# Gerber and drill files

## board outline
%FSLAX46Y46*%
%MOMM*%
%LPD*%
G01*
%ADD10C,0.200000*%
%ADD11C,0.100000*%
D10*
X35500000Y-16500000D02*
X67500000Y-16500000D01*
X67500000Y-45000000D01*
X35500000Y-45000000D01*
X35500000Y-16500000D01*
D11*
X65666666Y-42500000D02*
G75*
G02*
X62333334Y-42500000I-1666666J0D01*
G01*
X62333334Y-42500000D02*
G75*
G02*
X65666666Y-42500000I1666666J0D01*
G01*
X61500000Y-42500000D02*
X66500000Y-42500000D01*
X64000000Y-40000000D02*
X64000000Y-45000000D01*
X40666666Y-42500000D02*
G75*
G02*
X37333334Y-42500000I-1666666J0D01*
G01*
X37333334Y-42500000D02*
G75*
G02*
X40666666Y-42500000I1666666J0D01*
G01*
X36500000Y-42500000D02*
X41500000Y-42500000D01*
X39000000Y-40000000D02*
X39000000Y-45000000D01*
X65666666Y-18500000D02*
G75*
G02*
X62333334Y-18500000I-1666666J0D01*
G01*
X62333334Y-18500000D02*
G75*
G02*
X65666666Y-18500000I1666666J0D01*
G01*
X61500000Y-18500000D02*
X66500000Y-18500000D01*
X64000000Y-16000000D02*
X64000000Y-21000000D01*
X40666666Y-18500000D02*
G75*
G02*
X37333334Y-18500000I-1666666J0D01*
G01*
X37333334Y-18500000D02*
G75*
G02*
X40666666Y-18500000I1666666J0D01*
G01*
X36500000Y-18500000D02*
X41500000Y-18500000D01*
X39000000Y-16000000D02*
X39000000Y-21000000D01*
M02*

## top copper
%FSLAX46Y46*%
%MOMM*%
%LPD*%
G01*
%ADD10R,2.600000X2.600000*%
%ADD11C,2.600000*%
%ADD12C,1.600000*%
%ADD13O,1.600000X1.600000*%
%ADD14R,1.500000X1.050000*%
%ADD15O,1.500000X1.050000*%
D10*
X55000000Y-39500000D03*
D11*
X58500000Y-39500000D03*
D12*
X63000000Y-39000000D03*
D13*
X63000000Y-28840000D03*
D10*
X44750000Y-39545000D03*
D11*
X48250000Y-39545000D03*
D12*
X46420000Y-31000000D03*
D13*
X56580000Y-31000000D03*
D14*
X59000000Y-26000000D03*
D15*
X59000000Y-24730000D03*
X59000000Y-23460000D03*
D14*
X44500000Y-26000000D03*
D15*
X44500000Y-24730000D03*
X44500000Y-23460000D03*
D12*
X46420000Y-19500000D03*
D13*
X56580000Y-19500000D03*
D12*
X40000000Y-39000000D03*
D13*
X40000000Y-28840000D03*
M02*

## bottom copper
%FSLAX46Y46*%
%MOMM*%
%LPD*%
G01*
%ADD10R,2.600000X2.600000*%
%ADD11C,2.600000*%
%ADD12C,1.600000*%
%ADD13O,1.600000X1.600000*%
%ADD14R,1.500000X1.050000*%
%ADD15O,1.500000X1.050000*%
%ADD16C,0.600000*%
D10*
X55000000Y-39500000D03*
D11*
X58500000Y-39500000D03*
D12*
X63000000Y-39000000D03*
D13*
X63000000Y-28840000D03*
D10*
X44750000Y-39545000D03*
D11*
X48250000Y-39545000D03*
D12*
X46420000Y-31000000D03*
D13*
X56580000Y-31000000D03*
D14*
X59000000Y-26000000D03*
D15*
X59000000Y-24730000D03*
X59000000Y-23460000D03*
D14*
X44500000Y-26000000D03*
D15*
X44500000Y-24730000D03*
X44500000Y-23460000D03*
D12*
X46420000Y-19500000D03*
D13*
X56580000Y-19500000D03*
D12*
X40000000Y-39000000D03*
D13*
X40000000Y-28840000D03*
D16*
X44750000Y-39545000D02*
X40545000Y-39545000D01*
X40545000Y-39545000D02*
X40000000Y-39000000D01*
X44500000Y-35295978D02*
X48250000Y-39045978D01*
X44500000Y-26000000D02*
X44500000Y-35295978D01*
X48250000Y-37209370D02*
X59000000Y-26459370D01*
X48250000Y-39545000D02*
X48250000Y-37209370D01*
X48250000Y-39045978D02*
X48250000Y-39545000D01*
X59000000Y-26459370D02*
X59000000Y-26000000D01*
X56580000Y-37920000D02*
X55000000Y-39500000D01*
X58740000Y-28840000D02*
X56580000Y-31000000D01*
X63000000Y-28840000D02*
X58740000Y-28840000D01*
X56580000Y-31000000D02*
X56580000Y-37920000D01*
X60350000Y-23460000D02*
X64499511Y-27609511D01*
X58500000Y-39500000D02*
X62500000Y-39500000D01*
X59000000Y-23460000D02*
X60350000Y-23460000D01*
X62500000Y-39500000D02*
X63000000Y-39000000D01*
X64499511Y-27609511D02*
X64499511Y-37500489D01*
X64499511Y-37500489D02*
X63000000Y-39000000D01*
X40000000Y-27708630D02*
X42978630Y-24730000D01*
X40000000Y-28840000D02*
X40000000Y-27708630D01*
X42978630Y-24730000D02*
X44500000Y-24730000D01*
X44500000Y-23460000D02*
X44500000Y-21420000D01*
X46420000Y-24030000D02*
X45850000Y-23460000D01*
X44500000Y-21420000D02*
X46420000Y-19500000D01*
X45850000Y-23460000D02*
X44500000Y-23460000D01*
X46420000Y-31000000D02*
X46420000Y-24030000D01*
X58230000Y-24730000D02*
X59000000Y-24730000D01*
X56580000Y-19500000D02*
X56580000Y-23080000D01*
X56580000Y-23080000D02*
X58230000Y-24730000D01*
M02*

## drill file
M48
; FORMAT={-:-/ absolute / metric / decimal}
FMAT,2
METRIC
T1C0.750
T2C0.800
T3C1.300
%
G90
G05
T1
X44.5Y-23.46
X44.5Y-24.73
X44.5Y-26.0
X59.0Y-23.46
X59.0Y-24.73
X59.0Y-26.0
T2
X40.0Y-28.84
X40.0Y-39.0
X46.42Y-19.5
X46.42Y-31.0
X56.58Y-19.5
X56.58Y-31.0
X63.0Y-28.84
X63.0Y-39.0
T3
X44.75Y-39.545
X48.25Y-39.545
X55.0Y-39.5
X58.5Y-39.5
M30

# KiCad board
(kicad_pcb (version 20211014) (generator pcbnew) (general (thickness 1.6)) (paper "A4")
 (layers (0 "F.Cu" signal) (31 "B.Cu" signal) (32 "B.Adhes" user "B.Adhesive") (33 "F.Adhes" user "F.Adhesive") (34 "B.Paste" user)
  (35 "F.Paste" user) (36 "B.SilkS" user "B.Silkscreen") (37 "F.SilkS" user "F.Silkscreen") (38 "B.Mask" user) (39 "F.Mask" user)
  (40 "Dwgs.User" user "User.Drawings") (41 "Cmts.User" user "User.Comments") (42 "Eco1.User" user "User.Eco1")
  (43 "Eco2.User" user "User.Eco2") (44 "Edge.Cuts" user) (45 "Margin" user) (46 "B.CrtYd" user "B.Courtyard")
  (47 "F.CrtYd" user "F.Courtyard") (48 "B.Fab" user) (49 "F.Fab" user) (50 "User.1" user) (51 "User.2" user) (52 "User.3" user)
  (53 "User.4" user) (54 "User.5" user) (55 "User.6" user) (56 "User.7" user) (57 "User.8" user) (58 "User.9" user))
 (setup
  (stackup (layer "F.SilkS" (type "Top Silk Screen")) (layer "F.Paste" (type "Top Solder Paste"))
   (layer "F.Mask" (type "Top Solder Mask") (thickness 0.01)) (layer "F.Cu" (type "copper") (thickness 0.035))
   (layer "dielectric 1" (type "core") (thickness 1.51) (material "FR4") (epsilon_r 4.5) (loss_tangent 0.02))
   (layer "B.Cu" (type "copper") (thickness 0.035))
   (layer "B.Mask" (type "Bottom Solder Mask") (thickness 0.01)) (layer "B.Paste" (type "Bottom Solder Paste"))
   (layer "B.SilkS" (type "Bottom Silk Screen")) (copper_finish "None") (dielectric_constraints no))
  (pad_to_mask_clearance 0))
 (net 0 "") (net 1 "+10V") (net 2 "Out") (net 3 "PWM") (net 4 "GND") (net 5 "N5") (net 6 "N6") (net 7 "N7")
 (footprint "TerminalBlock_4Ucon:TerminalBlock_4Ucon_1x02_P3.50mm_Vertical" (layer "F.Cu") (at 55 39.5)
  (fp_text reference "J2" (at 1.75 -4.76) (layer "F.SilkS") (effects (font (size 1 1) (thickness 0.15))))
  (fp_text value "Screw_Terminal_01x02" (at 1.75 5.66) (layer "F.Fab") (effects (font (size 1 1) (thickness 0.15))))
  (pad "1" thru_hole rect locked (at 0 0) (size 2.6 2.6) (drill 1.3) (layers *.Cu *.Mask) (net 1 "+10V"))
  (pad "2" thru_hole circle locked (at 3.5 0) (size 2.6 2.6) (drill 1.3) (layers *.Cu *.Mask) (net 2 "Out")))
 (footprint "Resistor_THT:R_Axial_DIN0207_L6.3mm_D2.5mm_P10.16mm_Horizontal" (layer "F.Cu") (at 63 39 90)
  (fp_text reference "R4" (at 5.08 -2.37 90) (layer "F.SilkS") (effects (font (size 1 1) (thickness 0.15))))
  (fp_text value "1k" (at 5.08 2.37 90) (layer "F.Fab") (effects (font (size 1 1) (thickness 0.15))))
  (pad "1" thru_hole circle locked (at 0 0 90) (size 1.6 1.6) (drill 0.8) (layers *.Cu *.Mask) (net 2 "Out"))
  (pad "2" thru_hole oval locked (at 10.16 0 90) (size 1.6 1.6) (drill 0.8) (layers *.Cu *.Mask) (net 1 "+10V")))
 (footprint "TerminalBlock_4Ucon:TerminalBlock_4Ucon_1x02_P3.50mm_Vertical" (layer "F.Cu") (at 44.75 39.545)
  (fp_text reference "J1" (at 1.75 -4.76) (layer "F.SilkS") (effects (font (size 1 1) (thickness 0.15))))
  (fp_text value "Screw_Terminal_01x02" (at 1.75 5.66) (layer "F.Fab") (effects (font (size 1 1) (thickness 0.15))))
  (pad "1" thru_hole rect locked (at 0 0) (size 2.6 2.6) (drill 1.3) (layers *.Cu *.Mask) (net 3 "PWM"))
  (pad "2" thru_hole circle locked (at 3.5 0) (size 2.6 2.6) (drill 1.3) (layers *.Cu *.Mask) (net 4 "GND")))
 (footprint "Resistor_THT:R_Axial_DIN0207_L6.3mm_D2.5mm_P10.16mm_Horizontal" (layer "F.Cu") (at 46.42 31)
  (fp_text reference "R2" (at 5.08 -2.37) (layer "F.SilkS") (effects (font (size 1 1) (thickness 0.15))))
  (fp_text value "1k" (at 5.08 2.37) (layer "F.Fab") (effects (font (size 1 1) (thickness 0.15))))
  (pad "1" thru_hole circle locked (at 0 0) (size 1.6 1.6) (drill 0.8) (layers *.Cu *.Mask) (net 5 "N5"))
  (pad "2" thru_hole oval locked (at 10.16 0) (size 1.6 1.6) (drill 0.8) (layers *.Cu *.Mask) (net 1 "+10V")))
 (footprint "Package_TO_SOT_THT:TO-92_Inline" (layer "F.Cu") (at 59 26 90)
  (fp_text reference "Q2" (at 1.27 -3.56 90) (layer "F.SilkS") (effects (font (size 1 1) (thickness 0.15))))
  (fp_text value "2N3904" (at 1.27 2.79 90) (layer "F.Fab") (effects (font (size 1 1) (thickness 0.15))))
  (pad "1" thru_hole rect locked (at 0 0 90) (size 1.05 1.5) (drill 0.75) (layers *.Cu *.Mask) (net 4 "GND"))
  (pad "2" thru_hole oval locked (at 1.27 0 90) (size 1.05 1.5) (drill 0.75) (layers *.Cu *.Mask) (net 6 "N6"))
  (pad "3" thru_hole oval locked (at 2.54 0 90) (size 1.05 1.5) (drill 0.75) (layers *.Cu *.Mask) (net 2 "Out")))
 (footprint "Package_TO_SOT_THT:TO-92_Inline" (layer "F.Cu") (at 44.5 26 90)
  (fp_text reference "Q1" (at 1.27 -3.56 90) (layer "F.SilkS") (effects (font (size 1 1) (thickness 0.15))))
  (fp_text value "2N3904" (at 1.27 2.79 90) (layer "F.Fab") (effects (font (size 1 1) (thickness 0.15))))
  (pad "1" thru_hole rect locked (at 0 0 90) (size 1.05 1.5) (drill 0.75) (layers *.Cu *.Mask) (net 4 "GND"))
  (pad "2" thru_hole oval locked (at 1.27 0 90) (size 1.05 1.5) (drill 0.75) (layers *.Cu *.Mask) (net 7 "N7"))
  (pad "3" thru_hole oval locked (at 2.54 0 90) (size 1.05 1.5) (drill 0.75) (layers *.Cu *.Mask) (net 5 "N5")))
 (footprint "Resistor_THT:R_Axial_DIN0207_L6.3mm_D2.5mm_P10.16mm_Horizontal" (layer "F.Cu") (at 46.42 19.5)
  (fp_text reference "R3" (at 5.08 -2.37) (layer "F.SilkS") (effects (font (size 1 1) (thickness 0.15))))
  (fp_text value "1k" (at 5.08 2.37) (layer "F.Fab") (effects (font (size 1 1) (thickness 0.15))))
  (pad "1" thru_hole circle locked (at 0 0) (size 1.6 1.6) (drill 0.8) (layers *.Cu *.Mask) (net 5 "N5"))
  (pad "2" thru_hole oval locked (at 10.16 0) (size 1.6 1.6) (drill 0.8) (layers *.Cu *.Mask) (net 6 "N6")))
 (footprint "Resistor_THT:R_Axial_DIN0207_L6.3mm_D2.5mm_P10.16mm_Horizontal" (layer "F.Cu") (at 40 39 90)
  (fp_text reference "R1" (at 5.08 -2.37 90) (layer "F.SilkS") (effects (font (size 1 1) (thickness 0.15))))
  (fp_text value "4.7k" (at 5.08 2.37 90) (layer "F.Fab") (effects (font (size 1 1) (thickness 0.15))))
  (pad "1" thru_hole circle locked (at 0 0 90) (size 1.6 1.6) (drill 0.8) (layers *.Cu *.Mask) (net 3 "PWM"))
  (pad "2" thru_hole oval locked (at 10.16 0 90) (size 1.6 1.6) (drill 0.8) (layers *.Cu *.Mask) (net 7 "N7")))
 (gr_rect (start 67.5 45) (end 35.5 16.5) (layer "Edge.Cuts") (width 0.2) (fill none))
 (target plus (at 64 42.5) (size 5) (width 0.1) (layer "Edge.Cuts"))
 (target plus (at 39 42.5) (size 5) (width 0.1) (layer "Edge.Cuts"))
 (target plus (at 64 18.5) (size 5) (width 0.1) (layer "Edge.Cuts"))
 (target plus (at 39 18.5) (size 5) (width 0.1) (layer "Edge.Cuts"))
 (segment (start 44.75 39.545) (end 40.545 39.545) (width 0.6) (layer "B.Cu") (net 3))
 (segment (start 40.545 39.545) (end 40 39) (width 0.6) (layer "B.Cu") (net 3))
 (segment (start 44.5 35.295978) (end 48.25 39.045978) (width 0.6) (layer "B.Cu") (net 4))
 (segment (start 44.5 26) (end 44.5 35.295978) (width 0.6) (layer "B.Cu") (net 4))
 (segment (start 48.25 37.20937) (end 59 26.45937) (width 0.6) (layer "B.Cu") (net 4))
 (segment (start 48.25 39.545) (end 48.25 37.20937) (width 0.6) (layer "B.Cu") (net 4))
 (segment (start 48.25 39.045978) (end 48.25 39.545) (width 0.6) (layer "B.Cu") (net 4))
 (segment (start 59 26.45937) (end 59 26) (width 0.6) (layer "B.Cu") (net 4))
 (segment (start 56.58 37.92) (end 55 39.5) (width 0.6) (layer "B.Cu") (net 1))
 (segment (start 58.74 28.84) (end 56.58 31) (width 0.6) (layer "B.Cu") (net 1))
 (segment (start 63 28.84) (end 58.74 28.84) (width 0.6) (layer "B.Cu") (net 1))
 (segment (start 56.58 31) (end 56.58 37.92) (width 0.6) (layer "B.Cu") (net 1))
 (segment (start 60.35 23.46) (end 64.499511 27.609511) (width 0.6) (layer "B.Cu") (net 2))
 (segment (start 58.5 39.5) (end 62.5 39.5) (width 0.6) (layer "B.Cu") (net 2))
 (segment (start 59 23.46) (end 60.35 23.46) (width 0.6) (layer "B.Cu") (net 2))
 (segment (start 62.5 39.5) (end 63 39) (width 0.6) (layer "B.Cu") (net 2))
 (segment (start 64.499511 27.609511) (end 64.499511 37.500489) (width 0.6) (layer "B.Cu") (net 2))
 (segment (start 64.499511 37.500489) (end 63 39) (width 0.6) (layer "B.Cu") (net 2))
 (segment (start 40 27.70863) (end 42.97863 24.73) (width 0.6) (layer "B.Cu") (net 7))
 (segment (start 40 28.84) (end 40 27.70863) (width 0.6) (layer "B.Cu") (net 7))
 (segment (start 42.97863 24.73) (end 44.5 24.73) (width 0.6) (layer "B.Cu") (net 7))
 (segment (start 44.5 23.46) (end 44.5 21.42) (width 0.6) (layer "B.Cu") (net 5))
 (segment (start 46.42 24.03) (end 45.85 23.46) (width 0.6) (layer "B.Cu") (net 5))
 (segment (start 44.5 21.42) (end 46.42 19.5) (width 0.6) (layer "B.Cu") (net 5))
 (segment (start 45.85 23.46) (end 44.5 23.46) (width 0.6) (layer "B.Cu") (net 5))
 (segment (start 46.42 31) (end 46.42 24.03) (width 0.6) (layer "B.Cu") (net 5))
 (segment (start 58.23 24.73) (end 59 24.73) (width 0.6) (layer "B.Cu") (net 6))
 (segment (start 56.58 19.5) (end 56.58 23.08) (width 0.6) (layer "B.Cu") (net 6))
 (segment (start 56.58 23.08) (end 58.23 24.73) (width 0.6) (layer "B.Cu") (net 6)))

